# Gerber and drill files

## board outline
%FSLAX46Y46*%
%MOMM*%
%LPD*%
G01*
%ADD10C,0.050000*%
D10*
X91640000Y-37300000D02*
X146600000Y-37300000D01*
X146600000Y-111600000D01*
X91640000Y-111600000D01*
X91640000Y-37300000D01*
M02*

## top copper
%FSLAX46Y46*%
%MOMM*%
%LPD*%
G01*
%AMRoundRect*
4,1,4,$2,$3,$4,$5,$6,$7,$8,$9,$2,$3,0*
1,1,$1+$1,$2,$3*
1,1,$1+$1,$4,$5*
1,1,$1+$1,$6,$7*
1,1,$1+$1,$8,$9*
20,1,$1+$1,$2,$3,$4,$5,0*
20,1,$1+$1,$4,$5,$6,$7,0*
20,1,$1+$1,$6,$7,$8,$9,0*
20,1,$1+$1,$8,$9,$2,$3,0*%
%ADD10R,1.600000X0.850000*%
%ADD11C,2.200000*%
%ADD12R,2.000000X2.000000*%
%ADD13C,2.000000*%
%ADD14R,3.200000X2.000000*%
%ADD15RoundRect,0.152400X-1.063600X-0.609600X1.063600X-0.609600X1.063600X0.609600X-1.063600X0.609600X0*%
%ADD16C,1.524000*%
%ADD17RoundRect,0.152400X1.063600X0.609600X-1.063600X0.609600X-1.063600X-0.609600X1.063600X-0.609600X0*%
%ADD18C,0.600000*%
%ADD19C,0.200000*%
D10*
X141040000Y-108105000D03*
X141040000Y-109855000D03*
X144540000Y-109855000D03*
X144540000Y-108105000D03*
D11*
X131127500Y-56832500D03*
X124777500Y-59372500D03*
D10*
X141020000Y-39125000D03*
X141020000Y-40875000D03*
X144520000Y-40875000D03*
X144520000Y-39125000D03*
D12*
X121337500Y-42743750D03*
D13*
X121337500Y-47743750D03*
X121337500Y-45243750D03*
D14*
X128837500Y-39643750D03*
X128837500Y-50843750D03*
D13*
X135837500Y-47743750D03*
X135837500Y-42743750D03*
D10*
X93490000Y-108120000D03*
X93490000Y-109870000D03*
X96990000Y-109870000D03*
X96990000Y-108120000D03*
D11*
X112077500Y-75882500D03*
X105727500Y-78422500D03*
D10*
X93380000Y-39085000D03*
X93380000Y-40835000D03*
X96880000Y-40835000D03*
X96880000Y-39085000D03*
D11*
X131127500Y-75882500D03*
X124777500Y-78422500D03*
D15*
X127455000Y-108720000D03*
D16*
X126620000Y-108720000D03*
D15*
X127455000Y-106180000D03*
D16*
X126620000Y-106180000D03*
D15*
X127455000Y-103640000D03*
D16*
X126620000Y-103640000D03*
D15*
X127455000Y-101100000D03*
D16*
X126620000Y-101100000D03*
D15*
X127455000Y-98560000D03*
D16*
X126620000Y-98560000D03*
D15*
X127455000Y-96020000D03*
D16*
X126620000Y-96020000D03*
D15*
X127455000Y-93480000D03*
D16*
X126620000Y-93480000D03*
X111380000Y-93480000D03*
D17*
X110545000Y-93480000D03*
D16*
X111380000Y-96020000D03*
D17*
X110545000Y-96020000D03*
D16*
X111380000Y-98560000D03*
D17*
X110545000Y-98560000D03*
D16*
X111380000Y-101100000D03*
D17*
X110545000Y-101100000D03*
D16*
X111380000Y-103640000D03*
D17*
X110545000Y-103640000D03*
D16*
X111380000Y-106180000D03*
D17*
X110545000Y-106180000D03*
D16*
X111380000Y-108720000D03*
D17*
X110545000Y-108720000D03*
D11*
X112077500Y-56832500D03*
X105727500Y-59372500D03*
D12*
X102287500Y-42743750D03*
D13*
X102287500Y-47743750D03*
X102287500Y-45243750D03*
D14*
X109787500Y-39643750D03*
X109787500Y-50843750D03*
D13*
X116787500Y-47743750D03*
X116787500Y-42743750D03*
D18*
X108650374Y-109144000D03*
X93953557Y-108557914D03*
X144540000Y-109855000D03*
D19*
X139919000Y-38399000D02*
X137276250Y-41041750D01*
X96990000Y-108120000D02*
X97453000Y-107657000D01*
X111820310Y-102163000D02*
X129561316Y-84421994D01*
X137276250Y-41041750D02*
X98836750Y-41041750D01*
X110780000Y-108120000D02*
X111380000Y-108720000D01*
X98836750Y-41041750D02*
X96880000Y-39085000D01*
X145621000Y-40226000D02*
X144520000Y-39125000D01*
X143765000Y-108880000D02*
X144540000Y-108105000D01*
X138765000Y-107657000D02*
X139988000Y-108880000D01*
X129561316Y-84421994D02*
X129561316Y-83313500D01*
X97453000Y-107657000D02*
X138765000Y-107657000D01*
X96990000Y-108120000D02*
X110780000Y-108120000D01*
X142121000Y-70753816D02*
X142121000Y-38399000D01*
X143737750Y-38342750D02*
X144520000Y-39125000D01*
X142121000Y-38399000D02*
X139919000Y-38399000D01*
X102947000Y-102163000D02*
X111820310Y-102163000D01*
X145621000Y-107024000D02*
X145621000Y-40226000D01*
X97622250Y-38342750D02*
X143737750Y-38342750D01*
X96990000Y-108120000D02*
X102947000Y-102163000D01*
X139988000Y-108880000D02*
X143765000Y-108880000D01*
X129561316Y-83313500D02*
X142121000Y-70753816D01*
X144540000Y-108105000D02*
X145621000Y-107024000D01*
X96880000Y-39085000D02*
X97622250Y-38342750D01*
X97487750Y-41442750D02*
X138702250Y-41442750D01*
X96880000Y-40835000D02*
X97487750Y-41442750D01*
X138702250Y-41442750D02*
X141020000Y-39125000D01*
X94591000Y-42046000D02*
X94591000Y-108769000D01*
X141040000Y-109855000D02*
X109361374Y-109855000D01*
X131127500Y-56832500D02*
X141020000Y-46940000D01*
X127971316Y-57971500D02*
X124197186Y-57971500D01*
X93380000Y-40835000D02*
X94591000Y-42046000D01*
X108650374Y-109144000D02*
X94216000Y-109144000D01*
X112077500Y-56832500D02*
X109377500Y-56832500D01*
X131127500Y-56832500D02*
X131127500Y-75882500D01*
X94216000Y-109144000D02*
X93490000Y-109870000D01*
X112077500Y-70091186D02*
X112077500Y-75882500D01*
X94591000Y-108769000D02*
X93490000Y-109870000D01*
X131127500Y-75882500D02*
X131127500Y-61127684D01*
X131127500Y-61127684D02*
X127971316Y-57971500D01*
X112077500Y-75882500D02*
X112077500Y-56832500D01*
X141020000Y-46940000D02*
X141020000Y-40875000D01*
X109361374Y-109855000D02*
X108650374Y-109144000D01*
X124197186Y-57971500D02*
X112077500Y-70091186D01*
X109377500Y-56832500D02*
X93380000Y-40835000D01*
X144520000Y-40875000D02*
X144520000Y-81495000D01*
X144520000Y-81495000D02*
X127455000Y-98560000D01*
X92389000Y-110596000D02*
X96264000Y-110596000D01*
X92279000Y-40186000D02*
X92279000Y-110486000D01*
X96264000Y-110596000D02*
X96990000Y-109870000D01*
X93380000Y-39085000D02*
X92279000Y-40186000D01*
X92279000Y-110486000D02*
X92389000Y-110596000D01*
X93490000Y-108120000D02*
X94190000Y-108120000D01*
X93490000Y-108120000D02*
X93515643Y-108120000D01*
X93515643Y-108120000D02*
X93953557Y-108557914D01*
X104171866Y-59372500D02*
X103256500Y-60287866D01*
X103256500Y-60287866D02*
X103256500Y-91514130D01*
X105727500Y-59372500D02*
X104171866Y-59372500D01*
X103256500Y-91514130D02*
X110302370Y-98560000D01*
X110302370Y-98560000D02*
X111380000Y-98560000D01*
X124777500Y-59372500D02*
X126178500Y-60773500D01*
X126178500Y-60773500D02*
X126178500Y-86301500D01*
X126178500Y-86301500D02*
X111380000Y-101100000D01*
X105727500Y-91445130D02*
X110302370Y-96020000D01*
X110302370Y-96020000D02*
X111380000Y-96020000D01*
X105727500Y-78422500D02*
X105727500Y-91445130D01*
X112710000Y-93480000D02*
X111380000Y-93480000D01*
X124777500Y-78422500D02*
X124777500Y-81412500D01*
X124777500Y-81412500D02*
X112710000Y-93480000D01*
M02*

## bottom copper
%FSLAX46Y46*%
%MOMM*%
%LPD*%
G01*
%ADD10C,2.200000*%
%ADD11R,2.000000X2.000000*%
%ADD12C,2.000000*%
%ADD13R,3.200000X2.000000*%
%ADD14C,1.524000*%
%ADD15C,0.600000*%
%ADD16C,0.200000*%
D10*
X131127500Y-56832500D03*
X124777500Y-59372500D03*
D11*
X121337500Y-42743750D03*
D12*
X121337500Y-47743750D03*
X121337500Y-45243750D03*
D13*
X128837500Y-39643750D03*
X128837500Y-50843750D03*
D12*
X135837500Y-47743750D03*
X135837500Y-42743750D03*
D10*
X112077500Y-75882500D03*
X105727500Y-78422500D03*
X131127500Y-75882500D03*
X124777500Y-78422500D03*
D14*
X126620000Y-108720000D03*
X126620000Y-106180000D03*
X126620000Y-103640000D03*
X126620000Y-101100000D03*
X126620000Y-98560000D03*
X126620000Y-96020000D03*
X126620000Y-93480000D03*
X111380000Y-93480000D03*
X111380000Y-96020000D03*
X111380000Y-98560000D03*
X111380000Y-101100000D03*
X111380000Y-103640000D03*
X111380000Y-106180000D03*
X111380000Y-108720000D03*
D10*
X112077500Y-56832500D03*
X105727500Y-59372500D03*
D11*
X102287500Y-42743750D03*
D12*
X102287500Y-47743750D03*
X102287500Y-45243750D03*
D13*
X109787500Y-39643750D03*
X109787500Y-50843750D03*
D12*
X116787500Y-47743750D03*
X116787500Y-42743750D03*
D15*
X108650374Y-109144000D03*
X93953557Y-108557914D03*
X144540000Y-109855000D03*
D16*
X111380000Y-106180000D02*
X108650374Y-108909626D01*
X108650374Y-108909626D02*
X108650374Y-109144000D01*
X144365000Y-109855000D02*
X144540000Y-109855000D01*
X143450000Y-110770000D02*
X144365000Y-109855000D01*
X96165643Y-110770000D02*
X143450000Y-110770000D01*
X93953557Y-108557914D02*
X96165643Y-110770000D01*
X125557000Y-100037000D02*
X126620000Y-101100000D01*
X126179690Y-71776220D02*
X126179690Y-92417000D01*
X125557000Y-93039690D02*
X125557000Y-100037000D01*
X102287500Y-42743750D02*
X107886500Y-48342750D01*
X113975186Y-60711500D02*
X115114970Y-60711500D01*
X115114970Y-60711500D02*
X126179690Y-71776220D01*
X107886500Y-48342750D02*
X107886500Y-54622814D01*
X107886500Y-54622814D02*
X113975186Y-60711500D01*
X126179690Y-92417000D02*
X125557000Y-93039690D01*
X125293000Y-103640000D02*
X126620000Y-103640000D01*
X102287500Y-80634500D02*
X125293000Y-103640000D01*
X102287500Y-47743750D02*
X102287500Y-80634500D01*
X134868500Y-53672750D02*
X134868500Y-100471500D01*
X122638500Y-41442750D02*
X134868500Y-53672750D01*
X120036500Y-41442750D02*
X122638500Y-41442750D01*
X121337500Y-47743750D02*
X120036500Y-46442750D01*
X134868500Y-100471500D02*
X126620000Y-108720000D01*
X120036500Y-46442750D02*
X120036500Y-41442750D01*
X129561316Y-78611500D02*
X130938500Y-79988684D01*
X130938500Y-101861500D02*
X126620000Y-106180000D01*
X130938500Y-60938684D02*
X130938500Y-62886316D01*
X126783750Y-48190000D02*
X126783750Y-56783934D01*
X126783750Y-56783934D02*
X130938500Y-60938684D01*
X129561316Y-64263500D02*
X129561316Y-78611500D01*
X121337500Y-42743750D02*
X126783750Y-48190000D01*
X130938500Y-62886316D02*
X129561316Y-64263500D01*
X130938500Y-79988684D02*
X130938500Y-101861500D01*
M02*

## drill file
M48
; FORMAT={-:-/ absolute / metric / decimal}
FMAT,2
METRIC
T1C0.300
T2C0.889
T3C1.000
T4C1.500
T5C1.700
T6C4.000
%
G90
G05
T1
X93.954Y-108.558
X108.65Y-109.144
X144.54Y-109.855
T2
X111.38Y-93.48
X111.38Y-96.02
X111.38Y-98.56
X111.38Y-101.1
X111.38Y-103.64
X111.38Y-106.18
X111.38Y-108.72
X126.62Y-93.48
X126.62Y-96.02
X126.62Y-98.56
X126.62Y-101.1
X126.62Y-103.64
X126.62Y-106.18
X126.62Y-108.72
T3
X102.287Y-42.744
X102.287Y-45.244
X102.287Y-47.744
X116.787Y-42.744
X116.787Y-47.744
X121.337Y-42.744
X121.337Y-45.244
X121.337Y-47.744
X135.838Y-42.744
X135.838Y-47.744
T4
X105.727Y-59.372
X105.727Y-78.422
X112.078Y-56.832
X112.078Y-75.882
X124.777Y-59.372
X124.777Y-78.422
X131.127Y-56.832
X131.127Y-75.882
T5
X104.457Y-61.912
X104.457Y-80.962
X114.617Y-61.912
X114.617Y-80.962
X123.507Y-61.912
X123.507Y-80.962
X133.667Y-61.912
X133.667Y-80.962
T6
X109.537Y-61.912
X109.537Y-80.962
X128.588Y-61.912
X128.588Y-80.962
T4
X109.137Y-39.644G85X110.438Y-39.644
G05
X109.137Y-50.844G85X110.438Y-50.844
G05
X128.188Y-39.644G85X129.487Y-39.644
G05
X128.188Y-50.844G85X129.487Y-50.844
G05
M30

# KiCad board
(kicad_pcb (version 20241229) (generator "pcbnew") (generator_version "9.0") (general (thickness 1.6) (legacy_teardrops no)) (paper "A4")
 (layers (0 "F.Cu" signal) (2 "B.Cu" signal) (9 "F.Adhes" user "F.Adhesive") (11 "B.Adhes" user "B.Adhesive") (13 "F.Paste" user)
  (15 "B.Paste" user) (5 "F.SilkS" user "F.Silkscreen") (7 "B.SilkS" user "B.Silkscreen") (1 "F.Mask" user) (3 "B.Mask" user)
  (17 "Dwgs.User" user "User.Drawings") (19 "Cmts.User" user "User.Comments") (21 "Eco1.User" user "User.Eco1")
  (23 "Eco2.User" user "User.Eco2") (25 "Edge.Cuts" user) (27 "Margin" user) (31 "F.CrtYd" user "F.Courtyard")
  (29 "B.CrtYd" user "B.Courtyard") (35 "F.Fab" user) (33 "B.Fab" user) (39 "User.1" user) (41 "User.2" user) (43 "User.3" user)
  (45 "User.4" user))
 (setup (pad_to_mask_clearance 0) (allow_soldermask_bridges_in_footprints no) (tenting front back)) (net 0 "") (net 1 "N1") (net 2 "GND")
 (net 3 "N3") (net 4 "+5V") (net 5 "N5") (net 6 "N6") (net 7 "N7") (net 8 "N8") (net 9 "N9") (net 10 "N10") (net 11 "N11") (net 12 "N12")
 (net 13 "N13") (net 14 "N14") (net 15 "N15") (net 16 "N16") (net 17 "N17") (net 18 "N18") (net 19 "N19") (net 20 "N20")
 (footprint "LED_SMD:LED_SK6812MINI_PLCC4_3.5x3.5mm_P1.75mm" (layer "F.Cu") (at 142.79 108.98)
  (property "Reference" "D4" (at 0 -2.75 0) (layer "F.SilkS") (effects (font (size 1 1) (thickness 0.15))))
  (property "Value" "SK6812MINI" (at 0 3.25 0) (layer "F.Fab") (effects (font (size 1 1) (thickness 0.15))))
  (pad "1" smd rect (at -1.75 -0.875) (size 1.6 0.85) (layers "F.Cu" "F.Mask" "F.Paste") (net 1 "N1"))
  (pad "2" smd rect (at -1.75 0.875) (size 1.6 0.85) (layers "F.Cu" "F.Mask" "F.Paste") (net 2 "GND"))
  (pad "3" smd rect (at 1.75 0.875) (size 1.6 0.85) (layers "F.Cu" "F.Mask" "F.Paste") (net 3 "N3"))
  (pad "4" smd rect (at 1.75 -0.875) (size 1.6 0.85) (layers "F.Cu" "F.Mask" "F.Paste") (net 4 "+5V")))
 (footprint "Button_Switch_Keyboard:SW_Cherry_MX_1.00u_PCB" (layer "F.Cu") (at 131.1275 56.8325)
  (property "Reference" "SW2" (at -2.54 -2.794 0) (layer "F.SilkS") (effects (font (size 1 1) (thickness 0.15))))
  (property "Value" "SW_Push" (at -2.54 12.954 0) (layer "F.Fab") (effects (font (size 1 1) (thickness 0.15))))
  (pad "" np_thru_hole circle (at -7.62 5.08) (size 1.7 1.7) (drill 1.7) (layers "*.Cu" "*.Mask"))
  (pad "" np_thru_hole circle (at -2.54 5.08) (size 4 4) (drill 4) (layers "*.Cu" "*.Mask"))
  (pad "" np_thru_hole circle (at 2.54 5.08) (size 1.7 1.7) (drill 1.7) (layers "*.Cu" "*.Mask"))
  (pad "1" thru_hole circle (at 0 0) (size 2.2 2.2) (drill 1.5) (layers "*.Cu" "*.Mask") (remove_unused_layers no) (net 2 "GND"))
  (pad "2" thru_hole circle (at -6.35 2.54) (size 2.2 2.2) (drill 1.5) (layers "*.Cu" "*.Mask") (remove_unused_layers no) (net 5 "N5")))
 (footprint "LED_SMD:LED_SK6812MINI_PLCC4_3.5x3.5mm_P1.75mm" (layer "F.Cu") (at 142.77 40)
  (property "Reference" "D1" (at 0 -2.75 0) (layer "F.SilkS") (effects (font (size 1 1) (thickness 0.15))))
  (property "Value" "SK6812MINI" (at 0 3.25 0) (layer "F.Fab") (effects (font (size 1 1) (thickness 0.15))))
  (pad "1" smd rect (at -1.75 -0.875) (size 1.6 0.85) (layers "F.Cu" "F.Mask" "F.Paste") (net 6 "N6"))
  (pad "2" smd rect (at -1.75 0.875) (size 1.6 0.85) (layers "F.Cu" "F.Mask" "F.Paste") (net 2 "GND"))
  (pad "3" smd rect (at 1.75 0.875) (size 1.6 0.85) (layers "F.Cu" "F.Mask" "F.Paste") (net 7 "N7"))
  (pad "4" smd rect (at 1.75 -0.875) (size 1.6 0.85) (layers "F.Cu" "F.Mask" "F.Paste") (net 4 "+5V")))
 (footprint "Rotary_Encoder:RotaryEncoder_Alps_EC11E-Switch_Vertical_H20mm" (layer "F.Cu") (at 121.3375 42.74375)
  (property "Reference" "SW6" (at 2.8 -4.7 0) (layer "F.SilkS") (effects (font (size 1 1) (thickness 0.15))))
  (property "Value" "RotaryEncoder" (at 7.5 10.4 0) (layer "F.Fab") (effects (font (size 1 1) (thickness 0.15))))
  (pad "A" thru_hole rect (at 0 0) (size 2 2) (drill 1) (layers "*.Cu" "*.Mask") (remove_unused_layers no) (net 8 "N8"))
  (pad "B" thru_hole circle (at 0 5) (size 2 2) (drill 1) (layers "*.Cu" "*.Mask") (remove_unused_layers no) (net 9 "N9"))
  (pad "C" thru_hole circle (at 0 2.5) (size 2 2) (drill 1) (layers "*.Cu" "*.Mask") (remove_unused_layers no) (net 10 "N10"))
  (pad "MP" thru_hole rect (at 7.5 -3.1) (size 3.2 2) (drill oval 2.8 1.5) (layers "*.Cu" "*.Mask") (remove_unused_layers no))
  (pad "MP" thru_hole rect (at 7.5 8.1) (size 3.2 2) (drill oval 2.8 1.5) (layers "*.Cu" "*.Mask") (remove_unused_layers no))
  (pad "S1" thru_hole circle (at 14.5 5) (size 2 2) (drill 1) (layers "*.Cu" "*.Mask") (remove_unused_layers no))
  (pad "S2" thru_hole circle (at 14.5 0) (size 2 2) (drill 1) (layers "*.Cu" "*.Mask") (remove_unused_layers no)))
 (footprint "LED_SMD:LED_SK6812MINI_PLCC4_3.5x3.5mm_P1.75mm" (layer "F.Cu") (at 95.24 108.995)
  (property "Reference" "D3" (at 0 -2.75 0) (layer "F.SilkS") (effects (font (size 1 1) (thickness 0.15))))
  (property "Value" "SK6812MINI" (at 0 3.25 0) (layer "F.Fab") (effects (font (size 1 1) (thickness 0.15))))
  (pad "1" smd rect (at -1.75 -0.875) (size 1.6 0.85) (layers "F.Cu" "F.Mask" "F.Paste") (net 3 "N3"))
  (pad "2" smd rect (at -1.75 0.875) (size 1.6 0.85) (layers "F.Cu" "F.Mask" "F.Paste") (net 2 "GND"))
  (pad "3" smd rect (at 1.75 0.875) (size 1.6 0.85) (layers "F.Cu" "F.Mask" "F.Paste") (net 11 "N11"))
  (pad "4" smd rect (at 1.75 -0.875) (size 1.6 0.85) (layers "F.Cu" "F.Mask" "F.Paste") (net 4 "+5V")))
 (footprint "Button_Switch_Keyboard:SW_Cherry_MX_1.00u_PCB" (layer "F.Cu") (at 112.0775 75.8825)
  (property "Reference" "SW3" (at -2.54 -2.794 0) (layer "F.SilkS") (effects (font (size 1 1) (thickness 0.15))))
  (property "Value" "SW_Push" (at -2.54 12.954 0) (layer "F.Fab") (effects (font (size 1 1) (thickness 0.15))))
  (pad "" np_thru_hole circle (at -7.62 5.08) (size 1.7 1.7) (drill 1.7) (layers "*.Cu" "*.Mask"))
  (pad "" np_thru_hole circle (at -2.54 5.08) (size 4 4) (drill 4) (layers "*.Cu" "*.Mask"))
  (pad "" np_thru_hole circle (at 2.54 5.08) (size 1.7 1.7) (drill 1.7) (layers "*.Cu" "*.Mask"))
  (pad "1" thru_hole circle (at 0 0) (size 2.2 2.2) (drill 1.5) (layers "*.Cu" "*.Mask") (remove_unused_layers no) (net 2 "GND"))
  (pad "2" thru_hole circle (at -6.35 2.54) (size 2.2 2.2) (drill 1.5) (layers "*.Cu" "*.Mask") (remove_unused_layers no) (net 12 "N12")))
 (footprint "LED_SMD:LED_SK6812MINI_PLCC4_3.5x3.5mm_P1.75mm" (layer "F.Cu") (at 95.13 39.96)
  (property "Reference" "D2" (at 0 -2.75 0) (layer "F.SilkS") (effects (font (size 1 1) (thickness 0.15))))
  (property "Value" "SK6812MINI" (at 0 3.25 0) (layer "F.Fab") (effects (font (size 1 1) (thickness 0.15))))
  (pad "1" smd rect (at -1.75 -0.875) (size 1.6 0.85) (layers "F.Cu" "F.Mask" "F.Paste") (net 11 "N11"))
  (pad "2" smd rect (at -1.75 0.875) (size 1.6 0.85) (layers "F.Cu" "F.Mask" "F.Paste") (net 2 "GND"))
  (pad "3" smd rect (at 1.75 0.875) (size 1.6 0.85) (layers "F.Cu" "F.Mask" "F.Paste") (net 6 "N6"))
  (pad "4" smd rect (at 1.75 -0.875) (size 1.6 0.85) (layers "F.Cu" "F.Mask" "F.Paste") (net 4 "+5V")))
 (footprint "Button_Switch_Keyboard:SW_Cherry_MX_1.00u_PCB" (layer "F.Cu") (at 131.1275 75.8825)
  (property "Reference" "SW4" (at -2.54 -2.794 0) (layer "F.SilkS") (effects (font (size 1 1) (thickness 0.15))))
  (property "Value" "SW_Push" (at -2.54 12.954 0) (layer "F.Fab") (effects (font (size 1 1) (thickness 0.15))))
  (pad "" np_thru_hole circle (at -7.62 5.08) (size 1.7 1.7) (drill 1.7) (layers "*.Cu" "*.Mask"))
  (pad "" np_thru_hole circle (at -2.54 5.08) (size 4 4) (drill 4) (layers "*.Cu" "*.Mask"))
  (pad "" np_thru_hole circle (at 2.54 5.08) (size 1.7 1.7) (drill 1.7) (layers "*.Cu" "*.Mask"))
  (pad "1" thru_hole circle (at 0 0) (size 2.2 2.2) (drill 1.5) (layers "*.Cu" "*.Mask") (remove_unused_layers no) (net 2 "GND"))
  (pad "2" thru_hole circle (at -6.35 2.54) (size 2.2 2.2) (drill 1.5) (layers "*.Cu" "*.Mask") (remove_unused_layers no) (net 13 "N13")))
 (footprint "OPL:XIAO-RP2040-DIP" (layer "F.Cu") (at 119 101.1 180)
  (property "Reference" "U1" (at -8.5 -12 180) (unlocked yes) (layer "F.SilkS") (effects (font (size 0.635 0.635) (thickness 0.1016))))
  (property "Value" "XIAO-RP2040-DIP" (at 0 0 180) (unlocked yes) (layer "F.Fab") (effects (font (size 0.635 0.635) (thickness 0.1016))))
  (pad "1" smd roundrect (at -8.455 -7.62) (size 2.432 1.524) (layers "F.Cu" "F.Mask") (roundrect_rratio 0.1) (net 9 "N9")
   (thermal_bridge_angle 45))
  (pad "1" thru_hole circle (at -7.62 -7.62) (size 1.524 1.524) (drill 0.889) (layers "*.Cu" "*.Mask") (remove_unused_layers no)
   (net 9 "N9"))
  (pad "2" smd roundrect (at -8.455 -5.08) (size 2.432 1.524) (layers "F.Cu" "F.Mask") (roundrect_rratio 0.1) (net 8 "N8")
   (thermal_bridge_angle 45))
  (pad "2" thru_hole circle (at -7.62 -5.08) (size 1.524 1.524) (drill 0.889) (layers "*.Cu" "*.Mask") (remove_unused_layers no)
   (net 8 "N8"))
  (pad "3" smd roundrect (at -8.455 -2.54) (size 2.432 1.524) (layers "F.Cu" "F.Mask") (roundrect_rratio 0.1) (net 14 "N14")
   (thermal_bridge_angle 45))
  (pad "3" thru_hole circle (at -7.62 -2.54) (size 1.524 1.524) (drill 0.889) (layers "*.Cu" "*.Mask") (remove_unused_layers no)
   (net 14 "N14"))
  (pad "4" smd roundrect (at -8.455 0) (size 2.432 1.524) (layers "F.Cu" "F.Mask") (roundrect_rratio 0.1) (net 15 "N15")
   (thermal_bridge_angle 45))
  (pad "4" thru_hole circle (at -7.62 0) (size 1.524 1.524) (drill 0.889) (layers "*.Cu" "*.Mask") (remove_unused_layers no) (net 15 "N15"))
  (pad "5" smd roundrect (at -8.455 2.54) (size 2.432 1.524) (layers "F.Cu" "F.Mask") (roundrect_rratio 0.1) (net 7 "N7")
   (thermal_bridge_angle 45))
  (pad "5" thru_hole circle (at -7.62 2.54) (size 1.524 1.524) (drill 0.889) (layers "*.Cu" "*.Mask") (remove_unused_layers no) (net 7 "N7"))
  (pad "6" smd roundrect (at -8.455 5.08) (size 2.432 1.524) (layers "F.Cu" "F.Mask") (roundrect_rratio 0.1) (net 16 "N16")
   (thermal_bridge_angle 45))
  (pad "6" thru_hole circle (at -7.62 5.08) (size 1.524 1.524) (drill 0.889) (layers "*.Cu" "*.Mask") (remove_unused_layers no)
   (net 16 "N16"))
  (pad "7" smd roundrect (at -8.455 7.62) (size 2.432 1.524) (layers "F.Cu" "F.Mask") (roundrect_rratio 0.1) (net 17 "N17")
   (thermal_bridge_angle 45))
  (pad "7" thru_hole circle (at -7.62 7.62) (size 1.524 1.524) (drill 0.889) (layers "*.Cu" "*.Mask") (remove_unused_layers no)
   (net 17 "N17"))
  (pad "8" thru_hole circle (at 7.62 7.62 180) (size 1.524 1.524) (drill 0.889) (layers "*.Cu" "*.Mask") (remove_unused_layers no)
   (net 13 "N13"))
  (pad "8" smd roundrect (at 8.455 7.62 180) (size 2.432 1.524) (layers "F.Cu" "F.Mask") (roundrect_rratio 0.1) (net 13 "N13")
   (thermal_bridge_angle 45))
  (pad "9" thru_hole circle (at 7.62 5.08 180) (size 1.524 1.524) (drill 0.889) (layers "*.Cu" "*.Mask") (remove_unused_layers no)
   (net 12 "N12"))
  (pad "9" smd roundrect (at 8.455 5.08 180) (size 2.432 1.524) (layers "F.Cu" "F.Mask") (roundrect_rratio 0.1) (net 12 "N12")
   (thermal_bridge_angle 45))
  (pad "10" thru_hole circle (at 7.62 2.54 180) (size 1.524 1.524) (drill 0.889) (layers "*.Cu" "*.Mask") (remove_unused_layers no)
   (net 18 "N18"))
  (pad "10" smd roundrect (at 8.455 2.54 180) (size 2.432 1.524) (layers "F.Cu" "F.Mask") (roundrect_rratio 0.1) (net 18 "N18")
   (thermal_bridge_angle 45))
  (pad "11" thru_hole circle (at 7.62 0 180) (size 1.524 1.524) (drill 0.889) (layers "*.Cu" "*.Mask") (remove_unused_layers no)
   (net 5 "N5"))
  (pad "11" smd roundrect (at 8.455 0 180) (size 2.432 1.524) (layers "F.Cu" "F.Mask") (roundrect_rratio 0.1) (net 5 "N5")
   (thermal_bridge_angle 45))
  (pad "12" thru_hole circle (at 7.62 -2.54 180) (size 1.524 1.524) (drill 0.889) (layers "*.Cu" "*.Mask") (remove_unused_layers no)
   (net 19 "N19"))
  (pad "12" smd roundrect (at 8.455 -2.54 180) (size 2.432 1.524) (layers "F.Cu" "F.Mask") (roundrect_rratio 0.1) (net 19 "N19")
   (thermal_bridge_angle 45))
  (pad "13" thru_hole circle (at 7.62 -5.08 180) (size 1.524 1.524) (drill 0.889) (layers "*.Cu" "*.Mask") (remove_unused_layers no)
   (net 2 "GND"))
  (pad "13" smd roundrect (at 8.455 -5.08 180) (size 2.432 1.524) (layers "F.Cu" "F.Mask") (roundrect_rratio 0.1) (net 2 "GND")
   (thermal_bridge_angle 45))
  (pad "14" thru_hole circle (at 7.62 -7.62 180) (size 1.524 1.524) (drill 0.889) (layers "*.Cu" "*.Mask") (remove_unused_layers no)
   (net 4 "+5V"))
  (pad "14" smd roundrect (at 8.455 -7.62 180) (size 2.432 1.524) (layers "F.Cu" "F.Mask") (roundrect_rratio 0.1) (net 4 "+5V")
   (thermal_bridge_angle 45)))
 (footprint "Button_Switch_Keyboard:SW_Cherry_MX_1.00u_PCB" (layer "F.Cu") (at 112.0775 56.8325)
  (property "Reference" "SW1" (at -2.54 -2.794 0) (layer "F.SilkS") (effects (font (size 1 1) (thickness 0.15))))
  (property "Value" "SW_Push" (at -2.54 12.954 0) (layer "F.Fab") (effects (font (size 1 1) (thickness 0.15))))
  (pad "" np_thru_hole circle (at -7.62 5.08) (size 1.7 1.7) (drill 1.7) (layers "*.Cu" "*.Mask"))
  (pad "" np_thru_hole circle (at -2.54 5.08) (size 4 4) (drill 4) (layers "*.Cu" "*.Mask"))
  (pad "" np_thru_hole circle (at 2.54 5.08) (size 1.7 1.7) (drill 1.7) (layers "*.Cu" "*.Mask"))
  (pad "1" thru_hole circle (at 0 0) (size 2.2 2.2) (drill 1.5) (layers "*.Cu" "*.Mask") (remove_unused_layers no) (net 2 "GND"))
  (pad "2" thru_hole circle (at -6.35 2.54) (size 2.2 2.2) (drill 1.5) (layers "*.Cu" "*.Mask") (remove_unused_layers no) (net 18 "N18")))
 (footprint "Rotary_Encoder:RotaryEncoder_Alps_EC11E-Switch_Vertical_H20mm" (layer "F.Cu") (at 102.2875 42.74375)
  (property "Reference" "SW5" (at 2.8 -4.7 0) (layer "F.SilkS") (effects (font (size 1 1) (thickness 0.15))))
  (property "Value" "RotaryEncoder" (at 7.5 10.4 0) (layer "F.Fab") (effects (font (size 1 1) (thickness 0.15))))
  (pad "A" thru_hole rect (at 0 0) (size 2 2) (drill 1) (layers "*.Cu" "*.Mask") (remove_unused_layers no) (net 15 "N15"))
  (pad "B" thru_hole circle (at 0 5) (size 2 2) (drill 1) (layers "*.Cu" "*.Mask") (remove_unused_layers no) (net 14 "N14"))
  (pad "C" thru_hole circle (at 0 2.5) (size 2 2) (drill 1) (layers "*.Cu" "*.Mask") (remove_unused_layers no) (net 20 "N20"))
  (pad "MP" thru_hole rect (at 7.5 -3.1) (size 3.2 2) (drill oval 2.8 1.5) (layers "*.Cu" "*.Mask") (remove_unused_layers no))
  (pad "MP" thru_hole rect (at 7.5 8.1) (size 3.2 2) (drill oval 2.8 1.5) (layers "*.Cu" "*.Mask") (remove_unused_layers no))
  (pad "S1" thru_hole circle (at 14.5 5) (size 2 2) (drill 1) (layers "*.Cu" "*.Mask") (remove_unused_layers no))
  (pad "S2" thru_hole circle (at 14.5 0) (size 2 2) (drill 1) (layers "*.Cu" "*.Mask") (remove_unused_layers no)))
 (gr_rect (start 91.64 37.3) (end 146.6 111.6) (stroke (width 0.05) (type default)) (fill no) (layer "Edge.Cuts"))
 (segment (start 139.919 38.399) (end 137.27625 41.04175) (width 0.2) (layer "F.Cu") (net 4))
 (segment (start 96.99 108.12) (end 97.453 107.657) (width 0.2) (layer "F.Cu") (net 4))
 (segment (start 111.82031 102.163) (end 129.561316 84.421994) (width 0.2) (layer "F.Cu") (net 4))
 (segment (start 137.27625 41.04175) (end 98.83675 41.04175) (width 0.2) (layer "F.Cu") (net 4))
 (segment (start 110.78 108.12) (end 111.38 108.72) (width 0.2) (layer "F.Cu") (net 4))
 (segment (start 98.83675 41.04175) (end 96.88 39.085) (width 0.2) (layer "F.Cu") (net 4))
 (segment (start 145.621 40.226) (end 144.52 39.125) (width 0.2) (layer "F.Cu") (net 4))
 (segment (start 143.765 108.88) (end 144.54 108.105) (width 0.2) (layer "F.Cu") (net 4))
 (segment (start 138.765 107.657) (end 139.988 108.88) (width 0.2) (layer "F.Cu") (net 4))
 (segment (start 129.561316 84.421994) (end 129.561316 83.3135) (width 0.2) (layer "F.Cu") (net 4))
 (segment (start 97.453 107.657) (end 138.765 107.657) (width 0.2) (layer "F.Cu") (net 4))
 (segment (start 96.99 108.12) (end 110.78 108.12) (width 0.2) (layer "F.Cu") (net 4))
 (segment (start 142.121 70.753816) (end 142.121 38.399) (width 0.2) (layer "F.Cu") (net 4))
 (segment (start 143.73775 38.34275) (end 144.52 39.125) (width 0.2) (layer "F.Cu") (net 4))
 (segment (start 142.121 38.399) (end 139.919 38.399) (width 0.2) (layer "F.Cu") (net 4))
 (segment (start 102.947 102.163) (end 111.82031 102.163) (width 0.2) (layer "F.Cu") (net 4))
 (segment (start 145.621 107.024) (end 145.621 40.226) (width 0.2) (layer "F.Cu") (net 4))
 (segment (start 97.62225 38.34275) (end 143.73775 38.34275) (width 0.2) (layer "F.Cu") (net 4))
 (segment (start 96.99 108.12) (end 102.947 102.163) (width 0.2) (layer "F.Cu") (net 4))
 (segment (start 139.988 108.88) (end 143.765 108.88) (width 0.2) (layer "F.Cu") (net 4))
 (segment (start 129.561316 83.3135) (end 142.121 70.753816) (width 0.2) (layer "F.Cu") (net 4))
 (segment (start 144.54 108.105) (end 145.621 107.024) (width 0.2) (layer "F.Cu") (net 4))
 (segment (start 96.88 39.085) (end 97.62225 38.34275) (width 0.2) (layer "F.Cu") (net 4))
 (segment (start 97.48775 41.44275) (end 138.70225 41.44275) (width 0.2) (layer "F.Cu") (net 6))
 (segment (start 96.88 40.835) (end 97.48775 41.44275) (width 0.2) (layer "F.Cu") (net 6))
 (segment (start 138.70225 41.44275) (end 141.02 39.125) (width 0.2) (layer "F.Cu") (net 6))
 (segment (start 94.591 42.046) (end 94.591 108.769) (width 0.2) (layer "F.Cu") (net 2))
 (segment (start 141.04 109.855) (end 109.361374 109.855) (width 0.2) (layer "F.Cu") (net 2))
 (segment (start 131.1275 56.8325) (end 141.02 46.94) (width 0.2) (layer "F.Cu") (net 2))
 (segment (start 127.971316 57.9715) (end 124.197186 57.9715) (width 0.2) (layer "F.Cu") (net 2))
 (segment (start 93.38 40.835) (end 94.591 42.046) (width 0.2) (layer "F.Cu") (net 2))
 (segment (start 108.650374 109.144) (end 94.216 109.144) (width 0.2) (layer "F.Cu") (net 2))
 (segment (start 112.0775 56.8325) (end 109.3775 56.8325) (width 0.2) (layer "F.Cu") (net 2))
 (segment (start 131.1275 56.8325) (end 131.1275 75.8825) (width 0.2) (layer "F.Cu") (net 2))
 (segment (start 94.216 109.144) (end 93.49 109.87) (width 0.2) (layer "F.Cu") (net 2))
 (segment (start 112.0775 70.091186) (end 112.0775 75.8825) (width 0.2) (layer "F.Cu") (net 2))
 (segment (start 94.591 108.769) (end 93.49 109.87) (width 0.2) (layer "F.Cu") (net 2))
 (segment (start 131.1275 75.8825) (end 131.1275 61.127684) (width 0.2) (layer "F.Cu") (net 2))
 (segment (start 131.1275 61.127684) (end 127.971316 57.9715) (width 0.2) (layer "F.Cu") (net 2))
 (segment (start 112.0775 75.8825) (end 112.0775 56.8325) (width 0.2) (layer "F.Cu") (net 2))
 (segment (start 141.02 46.94) (end 141.02 40.875) (width 0.2) (layer "F.Cu") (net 2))
 (segment (start 109.361374 109.855) (end 108.650374 109.144) (width 0.2) (layer "F.Cu") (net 2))
 (segment (start 124.197186 57.9715) (end 112.0775 70.091186) (width 0.2) (layer "F.Cu") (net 2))
 (segment (start 109.3775 56.8325) (end 93.38 40.835) (width 0.2) (layer "F.Cu") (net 2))
 (via (at 108.650374 109.144) (size 0.6) (drill 0.3) (layers "F.Cu" "B.Cu") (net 2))
 (segment (start 111.38 106.18) (end 108.650374 108.909626) (width 0.2) (layer "B.Cu") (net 2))
 (segment (start 108.650374 108.909626) (end 108.650374 109.144) (width 0.2) (layer "B.Cu") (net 2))
 (segment (start 144.52 40.875) (end 144.52 81.495) (width 0.2) (layer "F.Cu") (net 7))
 (segment (start 144.52 81.495) (end 127.455 98.56) (width 0.2) (layer "F.Cu") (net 7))
 (segment (start 92.389 110.596) (end 96.264 110.596) (width 0.2) (layer "F.Cu") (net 11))
 (segment (start 92.279 40.186) (end 92.279 110.486) (width 0.2) (layer "F.Cu") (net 11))
 (segment (start 96.264 110.596) (end 96.99 109.87) (width 0.2) (layer "F.Cu") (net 11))
 (segment (start 93.38 39.085) (end 92.279 40.186) (width 0.2) (layer "F.Cu") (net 11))
 (segment (start 92.279 110.486) (end 92.389 110.596) (width 0.2) (layer "F.Cu") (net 11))
 (segment (start 93.49 108.12) (end 94.19 108.12) (width 0.2) (layer "F.Cu") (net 3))
 (segment (start 93.49 108.12) (end 93.515643 108.12) (width 0.2) (layer "F.Cu") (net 3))
 (segment (start 93.515643 108.12) (end 93.953557 108.557914) (width 0.2) (layer "F.Cu") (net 3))
 (via (at 93.953557 108.557914) (size 0.6) (drill 0.3) (layers "F.Cu" "B.Cu") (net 3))
 (via (at 144.54 109.855) (size 0.6) (drill 0.3) (layers "F.Cu" "B.Cu") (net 3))
 (segment (start 144.365 109.855) (end 144.54 109.855) (width 0.2) (layer "B.Cu") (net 3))
 (segment (start 143.45 110.77) (end 144.365 109.855) (width 0.2) (layer "B.Cu") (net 3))
 (segment (start 96.165643 110.77) (end 143.45 110.77) (width 0.2) (layer "B.Cu") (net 3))
 (segment (start 93.953557 108.557914) (end 96.165643 110.77) (width 0.2) (layer "B.Cu") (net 3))
 (segment (start 104.171866 59.3725) (end 103.2565 60.287866) (width 0.2) (layer "F.Cu") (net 18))
 (segment (start 103.2565 60.287866) (end 103.2565 91.51413) (width 0.2) (layer "F.Cu") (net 18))
 (segment (start 105.7275 59.3725) (end 104.171866 59.3725) (width 0.2) (layer "F.Cu") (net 18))
 (segment (start 103.2565 91.51413) (end 110.30237 98.56) (width 0.2) (layer "F.Cu") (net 18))
 (segment (start 110.30237 98.56) (end 111.38 98.56) (width 0.2) (layer "F.Cu") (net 18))
 (segment (start 124.7775 59.3725) (end 126.1785 60.7735) (width 0.2) (layer "F.Cu") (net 5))
 (segment (start 126.1785 60.7735) (end 126.1785 86.3015) (width 0.2) (layer "F.Cu") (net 5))
 (segment (start 126.1785 86.3015) (end 111.38 101.1) (width 0.2) (layer "F.Cu") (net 5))
 (segment (start 105.7275 91.44513) (end 110.30237 96.02) (width 0.2) (layer "F.Cu") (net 12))
 (segment (start 110.30237 96.02) (end 111.38 96.02) (width 0.2) (layer "F.Cu") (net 12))
 (segment (start 105.7275 78.4225) (end 105.7275 91.44513) (width 0.2) (layer "F.Cu") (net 12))
 (segment (start 112.71 93.48) (end 111.38 93.48) (width 0.2) (layer "F.Cu") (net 13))
 (segment (start 124.7775 78.4225) (end 124.7775 81.4125) (width 0.2) (layer "F.Cu") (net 13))
 (segment (start 124.7775 81.4125) (end 112.71 93.48) (width 0.2) (layer "F.Cu") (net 13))
 (segment (start 125.557 100.037) (end 126.62 101.1) (width 0.2) (layer "B.Cu") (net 15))
 (segment (start 126.17969 71.77622) (end 126.17969 92.417) (width 0.2) (layer "B.Cu") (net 15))
 (segment (start 125.557 93.03969) (end 125.557 100.037) (width 0.2) (layer "B.Cu") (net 15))
 (segment (start 102.2875 42.74375) (end 107.8865 48.34275) (width 0.2) (layer "B.Cu") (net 15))
 (segment (start 113.975186 60.7115) (end 115.11497 60.7115) (width 0.2) (layer "B.Cu") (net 15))
 (segment (start 115.11497 60.7115) (end 126.17969 71.77622) (width 0.2) (layer "B.Cu") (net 15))
 (segment (start 107.8865 48.34275) (end 107.8865 54.622814) (width 0.2) (layer "B.Cu") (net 15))
 (segment (start 107.8865 54.622814) (end 113.975186 60.7115) (width 0.2) (layer "B.Cu") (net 15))
 (segment (start 126.17969 92.417) (end 125.557 93.03969) (width 0.2) (layer "B.Cu") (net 15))
 (segment (start 125.293 103.64) (end 126.62 103.64) (width 0.2) (layer "B.Cu") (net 14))
 (segment (start 102.2875 80.6345) (end 125.293 103.64) (width 0.2) (layer "B.Cu") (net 14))
 (segment (start 102.2875 47.74375) (end 102.2875 80.6345) (width 0.2) (layer "B.Cu") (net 14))
 (segment (start 134.8685 53.67275) (end 134.8685 100.4715) (width 0.2) (layer "B.Cu") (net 9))
 (segment (start 122.6385 41.44275) (end 134.8685 53.67275) (width 0.2) (layer "B.Cu") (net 9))
 (segment (start 120.0365 41.44275) (end 122.6385 41.44275) (width 0.2) (layer "B.Cu") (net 9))
 (segment (start 121.3375 47.74375) (end 120.0365 46.44275) (width 0.2) (layer "B.Cu") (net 9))
 (segment (start 134.8685 100.4715) (end 126.62 108.72) (width 0.2) (layer "B.Cu") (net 9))
 (segment (start 120.0365 46.44275) (end 120.0365 41.44275) (width 0.2) (layer "B.Cu") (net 9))
 (segment (start 129.561316 78.6115) (end 130.9385 79.988684) (width 0.2) (layer "B.Cu") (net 8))
 (segment (start 130.9385 101.8615) (end 126.62 106.18) (width 0.2) (layer "B.Cu") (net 8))
 (segment (start 130.9385 60.938684) (end 130.9385 62.886316) (width 0.2) (layer "B.Cu") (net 8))
 (segment (start 126.78375 48.19) (end 126.78375 56.783934) (width 0.2) (layer "B.Cu") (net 8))
 (segment (start 126.78375 56.783934) (end 130.9385 60.938684) (width 0.2) (layer "B.Cu") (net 8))
 (segment (start 129.561316 64.2635) (end 129.561316 78.6115) (width 0.2) (layer "B.Cu") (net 8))
 (segment (start 121.3375 42.74375) (end 126.78375 48.19) (width 0.2) (layer "B.Cu") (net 8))
 (segment (start 130.9385 62.886316) (end 129.561316 64.2635) (width 0.2) (layer "B.Cu") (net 8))
 (segment (start 130.9385 79.988684) (end 130.9385 101.8615) (width 0.2) (layer "B.Cu") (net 8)))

